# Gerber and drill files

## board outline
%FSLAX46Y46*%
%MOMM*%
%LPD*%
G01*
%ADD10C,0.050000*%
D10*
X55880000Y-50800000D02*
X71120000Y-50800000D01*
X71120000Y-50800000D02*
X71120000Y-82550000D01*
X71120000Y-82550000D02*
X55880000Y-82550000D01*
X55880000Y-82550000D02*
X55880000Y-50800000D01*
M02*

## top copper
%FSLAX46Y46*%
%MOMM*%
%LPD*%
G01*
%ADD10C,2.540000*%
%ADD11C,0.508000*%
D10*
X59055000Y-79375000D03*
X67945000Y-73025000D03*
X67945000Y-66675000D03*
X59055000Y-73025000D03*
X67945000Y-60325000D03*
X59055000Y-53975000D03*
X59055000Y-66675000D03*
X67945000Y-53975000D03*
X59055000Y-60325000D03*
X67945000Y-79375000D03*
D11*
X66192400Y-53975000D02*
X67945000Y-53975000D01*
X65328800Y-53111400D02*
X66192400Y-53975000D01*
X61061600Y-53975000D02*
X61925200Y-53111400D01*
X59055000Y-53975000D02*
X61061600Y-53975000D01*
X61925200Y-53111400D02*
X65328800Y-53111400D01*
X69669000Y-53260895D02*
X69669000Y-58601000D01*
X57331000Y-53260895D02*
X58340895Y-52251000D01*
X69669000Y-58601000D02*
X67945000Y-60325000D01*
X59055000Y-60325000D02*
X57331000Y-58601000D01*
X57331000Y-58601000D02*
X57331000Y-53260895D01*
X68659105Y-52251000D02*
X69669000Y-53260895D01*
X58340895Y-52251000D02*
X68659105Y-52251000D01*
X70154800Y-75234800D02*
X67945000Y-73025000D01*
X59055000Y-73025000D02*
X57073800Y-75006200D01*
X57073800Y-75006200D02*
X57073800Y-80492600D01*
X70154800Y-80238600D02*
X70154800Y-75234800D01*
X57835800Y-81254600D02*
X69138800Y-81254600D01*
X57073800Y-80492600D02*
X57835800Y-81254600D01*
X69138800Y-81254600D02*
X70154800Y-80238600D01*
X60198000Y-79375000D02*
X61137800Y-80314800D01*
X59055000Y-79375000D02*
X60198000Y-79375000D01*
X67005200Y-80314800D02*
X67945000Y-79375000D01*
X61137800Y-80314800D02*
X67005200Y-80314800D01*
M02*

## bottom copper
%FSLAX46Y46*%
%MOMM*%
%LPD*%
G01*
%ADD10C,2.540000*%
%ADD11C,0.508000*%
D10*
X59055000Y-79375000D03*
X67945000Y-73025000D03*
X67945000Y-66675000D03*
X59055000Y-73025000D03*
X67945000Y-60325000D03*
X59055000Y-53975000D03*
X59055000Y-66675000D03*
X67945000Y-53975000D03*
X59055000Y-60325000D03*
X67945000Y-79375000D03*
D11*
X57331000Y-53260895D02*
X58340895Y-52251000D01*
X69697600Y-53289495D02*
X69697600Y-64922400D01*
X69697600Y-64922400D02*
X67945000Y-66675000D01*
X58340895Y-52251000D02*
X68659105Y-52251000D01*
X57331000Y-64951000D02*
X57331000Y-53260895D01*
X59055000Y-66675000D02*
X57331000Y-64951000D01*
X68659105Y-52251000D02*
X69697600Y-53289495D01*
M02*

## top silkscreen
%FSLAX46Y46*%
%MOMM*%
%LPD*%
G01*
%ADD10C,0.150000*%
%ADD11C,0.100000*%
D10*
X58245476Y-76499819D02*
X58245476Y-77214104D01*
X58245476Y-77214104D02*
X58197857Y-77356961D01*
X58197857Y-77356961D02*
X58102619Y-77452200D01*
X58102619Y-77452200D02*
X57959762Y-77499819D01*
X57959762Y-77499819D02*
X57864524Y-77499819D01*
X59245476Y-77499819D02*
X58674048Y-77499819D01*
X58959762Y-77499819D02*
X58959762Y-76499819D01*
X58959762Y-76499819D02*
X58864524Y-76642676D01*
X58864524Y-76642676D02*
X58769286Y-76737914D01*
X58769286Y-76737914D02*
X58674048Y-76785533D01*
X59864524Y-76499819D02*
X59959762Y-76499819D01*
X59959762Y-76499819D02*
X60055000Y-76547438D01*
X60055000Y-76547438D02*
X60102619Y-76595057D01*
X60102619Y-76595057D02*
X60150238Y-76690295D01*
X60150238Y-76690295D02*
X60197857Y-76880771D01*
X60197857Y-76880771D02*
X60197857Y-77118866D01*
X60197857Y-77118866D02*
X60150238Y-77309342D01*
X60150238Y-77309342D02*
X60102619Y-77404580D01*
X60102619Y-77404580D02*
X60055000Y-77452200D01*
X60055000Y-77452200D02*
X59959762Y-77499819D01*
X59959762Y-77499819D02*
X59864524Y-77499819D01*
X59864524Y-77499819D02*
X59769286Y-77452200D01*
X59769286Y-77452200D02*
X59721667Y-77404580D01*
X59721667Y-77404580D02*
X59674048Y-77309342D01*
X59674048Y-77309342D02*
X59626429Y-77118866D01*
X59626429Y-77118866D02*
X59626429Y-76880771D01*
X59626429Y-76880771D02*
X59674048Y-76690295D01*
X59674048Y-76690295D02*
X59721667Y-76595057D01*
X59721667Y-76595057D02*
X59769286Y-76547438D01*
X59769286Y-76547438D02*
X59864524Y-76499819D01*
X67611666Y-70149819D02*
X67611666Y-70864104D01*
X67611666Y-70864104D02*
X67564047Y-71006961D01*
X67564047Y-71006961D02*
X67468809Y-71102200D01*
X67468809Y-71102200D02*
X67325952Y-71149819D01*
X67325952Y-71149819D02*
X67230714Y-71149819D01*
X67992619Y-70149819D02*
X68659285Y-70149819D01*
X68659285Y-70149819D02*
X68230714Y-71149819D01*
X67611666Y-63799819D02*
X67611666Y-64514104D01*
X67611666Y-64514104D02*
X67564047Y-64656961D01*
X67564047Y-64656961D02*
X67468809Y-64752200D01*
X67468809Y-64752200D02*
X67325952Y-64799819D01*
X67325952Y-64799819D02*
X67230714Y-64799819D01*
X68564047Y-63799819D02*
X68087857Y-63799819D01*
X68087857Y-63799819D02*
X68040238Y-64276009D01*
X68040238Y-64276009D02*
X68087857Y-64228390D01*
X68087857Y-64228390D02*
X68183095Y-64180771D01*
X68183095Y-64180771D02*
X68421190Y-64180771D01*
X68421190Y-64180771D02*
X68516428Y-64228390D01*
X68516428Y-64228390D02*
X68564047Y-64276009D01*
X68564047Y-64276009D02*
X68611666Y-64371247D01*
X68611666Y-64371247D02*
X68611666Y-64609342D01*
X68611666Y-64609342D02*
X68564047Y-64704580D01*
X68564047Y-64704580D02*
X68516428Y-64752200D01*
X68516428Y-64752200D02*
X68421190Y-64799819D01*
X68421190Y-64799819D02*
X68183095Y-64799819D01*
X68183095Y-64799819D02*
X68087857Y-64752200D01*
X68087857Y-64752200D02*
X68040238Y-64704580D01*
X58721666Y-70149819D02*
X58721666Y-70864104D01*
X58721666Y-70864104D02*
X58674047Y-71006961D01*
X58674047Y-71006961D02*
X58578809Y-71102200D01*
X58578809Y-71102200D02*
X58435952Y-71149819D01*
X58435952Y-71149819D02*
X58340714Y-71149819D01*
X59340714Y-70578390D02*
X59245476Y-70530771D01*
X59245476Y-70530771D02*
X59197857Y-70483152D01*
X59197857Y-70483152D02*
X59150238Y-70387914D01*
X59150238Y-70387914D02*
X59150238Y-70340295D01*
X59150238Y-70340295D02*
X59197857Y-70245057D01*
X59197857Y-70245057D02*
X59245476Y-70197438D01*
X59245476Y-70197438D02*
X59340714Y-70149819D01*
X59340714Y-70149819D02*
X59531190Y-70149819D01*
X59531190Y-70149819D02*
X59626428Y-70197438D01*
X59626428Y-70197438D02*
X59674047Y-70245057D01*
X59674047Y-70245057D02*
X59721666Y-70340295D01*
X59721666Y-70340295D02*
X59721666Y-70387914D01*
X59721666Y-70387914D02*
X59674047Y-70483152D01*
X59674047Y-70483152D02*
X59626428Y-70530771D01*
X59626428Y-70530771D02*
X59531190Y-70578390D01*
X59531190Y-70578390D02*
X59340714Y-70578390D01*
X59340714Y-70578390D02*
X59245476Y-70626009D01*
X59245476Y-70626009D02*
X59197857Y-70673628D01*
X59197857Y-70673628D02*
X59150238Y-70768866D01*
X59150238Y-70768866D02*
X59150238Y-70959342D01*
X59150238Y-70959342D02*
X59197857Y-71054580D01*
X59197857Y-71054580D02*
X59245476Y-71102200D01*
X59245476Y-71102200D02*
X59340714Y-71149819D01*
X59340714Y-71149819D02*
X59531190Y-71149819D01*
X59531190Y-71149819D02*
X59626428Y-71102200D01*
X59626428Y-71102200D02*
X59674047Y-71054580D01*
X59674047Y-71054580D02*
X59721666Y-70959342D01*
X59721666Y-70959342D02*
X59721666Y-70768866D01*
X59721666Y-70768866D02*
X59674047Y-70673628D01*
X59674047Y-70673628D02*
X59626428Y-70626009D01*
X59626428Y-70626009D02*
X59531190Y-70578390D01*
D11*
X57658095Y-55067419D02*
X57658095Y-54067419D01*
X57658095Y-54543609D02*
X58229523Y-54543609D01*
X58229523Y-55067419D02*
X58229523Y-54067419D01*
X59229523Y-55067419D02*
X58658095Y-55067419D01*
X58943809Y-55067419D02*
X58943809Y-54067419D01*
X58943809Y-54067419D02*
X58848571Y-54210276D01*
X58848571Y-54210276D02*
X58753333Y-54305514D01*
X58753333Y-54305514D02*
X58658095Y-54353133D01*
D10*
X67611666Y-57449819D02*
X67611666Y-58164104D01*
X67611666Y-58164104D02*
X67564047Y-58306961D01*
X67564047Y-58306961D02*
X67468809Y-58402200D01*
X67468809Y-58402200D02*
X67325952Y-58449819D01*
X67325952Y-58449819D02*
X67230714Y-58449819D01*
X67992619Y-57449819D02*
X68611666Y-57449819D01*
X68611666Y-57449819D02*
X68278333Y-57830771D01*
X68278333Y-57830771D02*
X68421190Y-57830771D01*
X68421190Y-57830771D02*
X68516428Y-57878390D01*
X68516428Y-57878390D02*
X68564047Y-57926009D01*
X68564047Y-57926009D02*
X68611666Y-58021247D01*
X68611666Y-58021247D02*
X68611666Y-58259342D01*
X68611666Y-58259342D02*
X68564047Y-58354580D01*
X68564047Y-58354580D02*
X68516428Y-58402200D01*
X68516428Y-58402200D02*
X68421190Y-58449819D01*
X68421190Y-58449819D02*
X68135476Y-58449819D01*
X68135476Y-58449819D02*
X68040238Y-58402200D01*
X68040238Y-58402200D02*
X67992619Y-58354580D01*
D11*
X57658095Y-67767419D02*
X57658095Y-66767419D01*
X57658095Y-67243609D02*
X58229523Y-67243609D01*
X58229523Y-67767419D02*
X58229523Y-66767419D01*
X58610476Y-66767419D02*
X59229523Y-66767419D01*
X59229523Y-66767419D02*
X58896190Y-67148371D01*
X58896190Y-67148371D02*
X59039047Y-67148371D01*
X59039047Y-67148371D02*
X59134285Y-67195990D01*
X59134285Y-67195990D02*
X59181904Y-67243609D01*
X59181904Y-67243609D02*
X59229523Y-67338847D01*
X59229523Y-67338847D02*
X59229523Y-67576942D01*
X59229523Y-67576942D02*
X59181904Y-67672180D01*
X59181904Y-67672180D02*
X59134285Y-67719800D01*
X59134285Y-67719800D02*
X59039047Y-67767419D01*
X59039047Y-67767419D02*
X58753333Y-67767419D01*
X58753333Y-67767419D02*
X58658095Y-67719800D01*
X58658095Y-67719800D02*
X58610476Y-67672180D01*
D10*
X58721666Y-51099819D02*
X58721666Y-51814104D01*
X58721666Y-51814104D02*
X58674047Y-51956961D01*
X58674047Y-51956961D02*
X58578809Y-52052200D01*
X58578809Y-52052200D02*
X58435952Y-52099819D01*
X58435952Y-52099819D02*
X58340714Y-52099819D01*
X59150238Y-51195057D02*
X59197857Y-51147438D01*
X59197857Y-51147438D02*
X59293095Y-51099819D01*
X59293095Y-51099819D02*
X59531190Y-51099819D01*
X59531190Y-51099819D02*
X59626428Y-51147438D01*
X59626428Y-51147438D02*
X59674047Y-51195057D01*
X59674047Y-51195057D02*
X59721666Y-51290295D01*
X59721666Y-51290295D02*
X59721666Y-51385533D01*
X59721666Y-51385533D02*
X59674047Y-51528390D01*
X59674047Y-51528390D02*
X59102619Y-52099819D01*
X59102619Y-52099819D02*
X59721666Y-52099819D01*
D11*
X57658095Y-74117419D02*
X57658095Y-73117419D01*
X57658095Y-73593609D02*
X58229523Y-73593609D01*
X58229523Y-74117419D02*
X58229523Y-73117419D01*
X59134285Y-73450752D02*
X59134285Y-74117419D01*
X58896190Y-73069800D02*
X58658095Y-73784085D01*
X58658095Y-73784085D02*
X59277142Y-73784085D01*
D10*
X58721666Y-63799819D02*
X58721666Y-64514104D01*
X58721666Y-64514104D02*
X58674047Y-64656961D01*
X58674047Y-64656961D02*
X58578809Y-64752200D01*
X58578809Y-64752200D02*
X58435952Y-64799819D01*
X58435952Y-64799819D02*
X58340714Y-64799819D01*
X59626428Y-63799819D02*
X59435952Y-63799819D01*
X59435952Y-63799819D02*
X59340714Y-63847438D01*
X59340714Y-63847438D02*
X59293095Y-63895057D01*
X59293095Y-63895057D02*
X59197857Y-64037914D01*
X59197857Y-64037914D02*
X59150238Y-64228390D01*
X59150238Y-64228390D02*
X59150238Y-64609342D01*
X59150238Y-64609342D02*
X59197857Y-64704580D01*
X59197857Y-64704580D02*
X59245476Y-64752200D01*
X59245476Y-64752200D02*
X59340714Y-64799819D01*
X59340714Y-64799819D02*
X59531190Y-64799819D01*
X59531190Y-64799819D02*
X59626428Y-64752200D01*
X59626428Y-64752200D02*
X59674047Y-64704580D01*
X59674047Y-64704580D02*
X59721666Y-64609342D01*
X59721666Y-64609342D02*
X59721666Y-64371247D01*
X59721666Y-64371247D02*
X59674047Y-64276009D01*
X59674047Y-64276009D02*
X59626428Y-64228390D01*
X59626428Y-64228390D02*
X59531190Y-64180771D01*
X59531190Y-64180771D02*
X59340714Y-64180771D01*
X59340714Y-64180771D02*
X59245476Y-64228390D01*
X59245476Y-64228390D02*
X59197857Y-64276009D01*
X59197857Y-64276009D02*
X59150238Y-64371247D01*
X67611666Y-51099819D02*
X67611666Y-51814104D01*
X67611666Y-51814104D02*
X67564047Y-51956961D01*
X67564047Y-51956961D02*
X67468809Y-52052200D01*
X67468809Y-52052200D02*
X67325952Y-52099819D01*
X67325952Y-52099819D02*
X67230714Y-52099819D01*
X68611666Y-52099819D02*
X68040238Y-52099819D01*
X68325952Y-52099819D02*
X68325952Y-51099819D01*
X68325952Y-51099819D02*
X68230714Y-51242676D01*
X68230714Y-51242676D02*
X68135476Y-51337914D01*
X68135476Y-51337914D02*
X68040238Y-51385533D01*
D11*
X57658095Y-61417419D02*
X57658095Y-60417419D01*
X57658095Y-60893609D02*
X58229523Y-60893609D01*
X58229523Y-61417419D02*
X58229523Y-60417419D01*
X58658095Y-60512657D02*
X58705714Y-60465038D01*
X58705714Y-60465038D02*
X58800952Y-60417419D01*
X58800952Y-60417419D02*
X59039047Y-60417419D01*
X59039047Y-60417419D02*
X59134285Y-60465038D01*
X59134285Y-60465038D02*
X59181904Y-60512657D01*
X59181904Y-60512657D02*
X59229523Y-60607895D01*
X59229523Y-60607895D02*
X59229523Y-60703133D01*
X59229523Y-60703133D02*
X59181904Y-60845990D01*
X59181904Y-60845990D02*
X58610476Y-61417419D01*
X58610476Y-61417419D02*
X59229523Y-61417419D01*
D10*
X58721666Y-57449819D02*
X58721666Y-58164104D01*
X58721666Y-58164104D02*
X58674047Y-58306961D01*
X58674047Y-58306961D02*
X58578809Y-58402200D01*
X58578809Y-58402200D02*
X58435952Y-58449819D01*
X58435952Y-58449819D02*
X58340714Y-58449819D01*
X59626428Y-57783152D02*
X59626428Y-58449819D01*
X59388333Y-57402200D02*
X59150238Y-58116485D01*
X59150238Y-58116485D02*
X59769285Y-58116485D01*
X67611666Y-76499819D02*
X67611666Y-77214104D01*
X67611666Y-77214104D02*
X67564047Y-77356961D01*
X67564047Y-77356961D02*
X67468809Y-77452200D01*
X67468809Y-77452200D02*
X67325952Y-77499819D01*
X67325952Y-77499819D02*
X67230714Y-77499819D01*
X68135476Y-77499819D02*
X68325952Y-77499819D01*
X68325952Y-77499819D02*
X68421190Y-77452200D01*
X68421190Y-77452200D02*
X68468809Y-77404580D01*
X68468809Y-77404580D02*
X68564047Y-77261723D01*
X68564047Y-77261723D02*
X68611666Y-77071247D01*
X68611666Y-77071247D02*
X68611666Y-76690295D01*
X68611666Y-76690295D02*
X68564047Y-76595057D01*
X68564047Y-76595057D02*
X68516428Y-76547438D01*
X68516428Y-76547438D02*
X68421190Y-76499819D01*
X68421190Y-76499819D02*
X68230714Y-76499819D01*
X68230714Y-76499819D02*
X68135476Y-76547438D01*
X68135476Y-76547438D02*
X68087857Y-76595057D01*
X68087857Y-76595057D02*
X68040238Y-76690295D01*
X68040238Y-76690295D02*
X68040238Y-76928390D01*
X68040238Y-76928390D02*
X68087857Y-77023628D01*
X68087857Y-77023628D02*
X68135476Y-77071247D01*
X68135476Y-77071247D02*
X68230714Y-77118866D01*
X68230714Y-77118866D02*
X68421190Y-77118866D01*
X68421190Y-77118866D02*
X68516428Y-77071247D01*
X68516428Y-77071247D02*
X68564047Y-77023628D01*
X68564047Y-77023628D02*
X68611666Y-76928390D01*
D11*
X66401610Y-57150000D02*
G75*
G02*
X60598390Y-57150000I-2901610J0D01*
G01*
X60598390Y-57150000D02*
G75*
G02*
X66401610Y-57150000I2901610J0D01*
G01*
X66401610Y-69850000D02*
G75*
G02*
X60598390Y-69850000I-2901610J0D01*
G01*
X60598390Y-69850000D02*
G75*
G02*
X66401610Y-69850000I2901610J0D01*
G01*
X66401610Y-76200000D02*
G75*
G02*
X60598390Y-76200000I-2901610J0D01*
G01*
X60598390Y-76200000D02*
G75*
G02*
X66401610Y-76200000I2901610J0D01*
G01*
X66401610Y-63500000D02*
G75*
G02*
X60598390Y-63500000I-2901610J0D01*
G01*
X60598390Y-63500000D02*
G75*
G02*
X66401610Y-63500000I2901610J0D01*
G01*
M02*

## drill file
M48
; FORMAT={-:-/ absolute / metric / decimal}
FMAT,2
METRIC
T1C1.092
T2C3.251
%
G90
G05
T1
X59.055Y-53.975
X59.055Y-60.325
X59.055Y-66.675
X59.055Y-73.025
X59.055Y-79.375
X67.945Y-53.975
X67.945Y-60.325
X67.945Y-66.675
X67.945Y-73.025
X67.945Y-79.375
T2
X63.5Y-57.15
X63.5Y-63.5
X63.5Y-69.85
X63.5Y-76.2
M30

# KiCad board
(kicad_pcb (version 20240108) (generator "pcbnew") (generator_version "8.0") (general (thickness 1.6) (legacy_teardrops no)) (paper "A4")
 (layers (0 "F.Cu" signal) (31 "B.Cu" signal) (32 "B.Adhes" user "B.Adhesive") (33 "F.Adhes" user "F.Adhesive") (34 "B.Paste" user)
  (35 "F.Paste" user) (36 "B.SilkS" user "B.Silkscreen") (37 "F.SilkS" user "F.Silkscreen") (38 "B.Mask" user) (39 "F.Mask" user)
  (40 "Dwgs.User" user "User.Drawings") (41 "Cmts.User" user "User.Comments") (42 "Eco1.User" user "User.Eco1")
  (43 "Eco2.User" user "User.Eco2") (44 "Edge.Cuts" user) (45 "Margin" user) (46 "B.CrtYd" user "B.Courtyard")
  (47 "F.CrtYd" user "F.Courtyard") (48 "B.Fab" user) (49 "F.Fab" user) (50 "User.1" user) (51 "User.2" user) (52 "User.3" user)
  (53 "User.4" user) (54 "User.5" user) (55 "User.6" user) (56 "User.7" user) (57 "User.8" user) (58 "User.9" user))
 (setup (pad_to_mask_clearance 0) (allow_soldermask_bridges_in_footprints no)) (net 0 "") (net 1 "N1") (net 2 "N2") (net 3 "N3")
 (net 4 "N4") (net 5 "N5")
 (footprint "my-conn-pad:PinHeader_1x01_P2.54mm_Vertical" (layer "F.Cu") (at 59.055 79.375)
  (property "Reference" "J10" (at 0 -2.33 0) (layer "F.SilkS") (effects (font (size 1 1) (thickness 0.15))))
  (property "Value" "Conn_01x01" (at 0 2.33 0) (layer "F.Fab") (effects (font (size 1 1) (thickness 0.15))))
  (pad "1" thru_hole circle (at 0 0) (size 2.54 2.54) (drill 1.0922) (layers "*.Cu" "*.Mask") (remove_unused_layers no) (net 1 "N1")))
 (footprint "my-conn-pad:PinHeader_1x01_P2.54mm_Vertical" (layer "F.Cu") (at 67.945 73.025)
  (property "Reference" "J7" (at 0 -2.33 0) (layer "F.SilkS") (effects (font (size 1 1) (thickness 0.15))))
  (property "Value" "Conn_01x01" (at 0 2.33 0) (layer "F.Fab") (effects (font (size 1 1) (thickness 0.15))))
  (pad "1" thru_hole circle (at 0 0) (size 2.54 2.54) (drill 1.0922) (layers "*.Cu" "*.Mask") (remove_unused_layers no) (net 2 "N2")))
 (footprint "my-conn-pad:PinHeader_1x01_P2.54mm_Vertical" (layer "F.Cu") (at 67.945 66.675)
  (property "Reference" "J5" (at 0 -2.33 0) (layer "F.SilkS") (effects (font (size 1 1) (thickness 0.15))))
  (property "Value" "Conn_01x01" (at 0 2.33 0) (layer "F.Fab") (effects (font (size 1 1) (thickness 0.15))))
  (pad "1" thru_hole circle (at 0 0) (size 2.54 2.54) (drill 1.0922) (layers "*.Cu" "*.Mask") (remove_unused_layers no) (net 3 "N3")))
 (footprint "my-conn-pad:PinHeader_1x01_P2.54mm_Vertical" (layer "F.Cu") (at 59.055 73.025)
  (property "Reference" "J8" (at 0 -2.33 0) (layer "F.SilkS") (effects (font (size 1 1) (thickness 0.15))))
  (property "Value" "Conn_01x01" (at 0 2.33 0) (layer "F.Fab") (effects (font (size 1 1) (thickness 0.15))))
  (pad "1" thru_hole circle (at 0 0) (size 2.54 2.54) (drill 1.0922) (layers "*.Cu" "*.Mask") (remove_unused_layers no) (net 2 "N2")))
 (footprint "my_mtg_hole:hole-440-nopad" (layer "F.Cu") (at 63.5 57.15)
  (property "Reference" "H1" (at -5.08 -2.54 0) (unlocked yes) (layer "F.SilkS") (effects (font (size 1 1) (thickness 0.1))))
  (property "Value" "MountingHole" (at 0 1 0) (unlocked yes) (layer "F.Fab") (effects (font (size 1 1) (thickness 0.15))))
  (fp_circle (center 0 0) (end 1.143 2.667) (stroke (width 0.1) (type default)) (fill none) (layer "F.SilkS"))
  (pad "" np_thru_hole circle (at 0 0) (size 1.524 1.524) (drill 3.2512) (layers "F&B.Cu" "*.Mask")))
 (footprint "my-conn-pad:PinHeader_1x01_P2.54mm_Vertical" (layer "F.Cu") (at 67.945 60.325)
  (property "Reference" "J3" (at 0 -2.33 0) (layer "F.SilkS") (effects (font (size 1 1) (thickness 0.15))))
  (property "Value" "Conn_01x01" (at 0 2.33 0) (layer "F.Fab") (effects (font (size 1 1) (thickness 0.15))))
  (pad "1" thru_hole circle (at 0 0) (size 2.54 2.54) (drill 1.0922) (layers "*.Cu" "*.Mask") (remove_unused_layers no) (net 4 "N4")))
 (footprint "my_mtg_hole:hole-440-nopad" (layer "F.Cu") (at 63.5 69.85)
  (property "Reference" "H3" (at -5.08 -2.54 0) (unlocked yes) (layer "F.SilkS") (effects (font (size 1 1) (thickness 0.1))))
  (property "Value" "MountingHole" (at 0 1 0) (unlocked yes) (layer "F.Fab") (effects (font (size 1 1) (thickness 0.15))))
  (fp_circle (center 0 0) (end 1.143 2.667) (stroke (width 0.1) (type default)) (fill none) (layer "F.SilkS"))
  (pad "" np_thru_hole circle (at 0 0) (size 1.524 1.524) (drill 3.2512) (layers "F&B.Cu" "*.Mask")))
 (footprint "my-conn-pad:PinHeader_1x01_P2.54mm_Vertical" (layer "F.Cu") (at 59.055 53.975)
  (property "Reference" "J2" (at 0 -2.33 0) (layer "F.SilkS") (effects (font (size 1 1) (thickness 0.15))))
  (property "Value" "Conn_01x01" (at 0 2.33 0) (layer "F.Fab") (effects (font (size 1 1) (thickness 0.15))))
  (pad "1" thru_hole circle (at 0 0) (size 2.54 2.54) (drill 1.0922) (layers "*.Cu" "*.Mask") (remove_unused_layers no) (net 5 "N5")))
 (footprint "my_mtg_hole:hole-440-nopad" (layer "F.Cu") (at 63.5 76.2)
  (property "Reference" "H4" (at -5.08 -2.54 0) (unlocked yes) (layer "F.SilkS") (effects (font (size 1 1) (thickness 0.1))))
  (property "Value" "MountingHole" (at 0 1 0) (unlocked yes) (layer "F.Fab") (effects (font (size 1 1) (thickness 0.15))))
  (fp_circle (center 0 0) (end 1.143 2.667) (stroke (width 0.1) (type default)) (fill none) (layer "F.SilkS"))
  (pad "" np_thru_hole circle (at 0 0) (size 1.524 1.524) (drill 3.2512) (layers "F&B.Cu" "*.Mask")))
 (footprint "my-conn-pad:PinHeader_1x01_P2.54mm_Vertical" (layer "F.Cu") (at 59.055 66.675)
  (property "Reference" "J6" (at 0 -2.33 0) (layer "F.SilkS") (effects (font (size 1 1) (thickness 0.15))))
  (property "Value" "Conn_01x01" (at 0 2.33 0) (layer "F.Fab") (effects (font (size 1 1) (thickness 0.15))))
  (pad "1" thru_hole circle (at 0 0) (size 2.54 2.54) (drill 1.0922) (layers "*.Cu" "*.Mask") (remove_unused_layers no) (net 3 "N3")))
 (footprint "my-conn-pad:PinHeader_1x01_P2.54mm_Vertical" (layer "F.Cu") (at 67.945 53.975)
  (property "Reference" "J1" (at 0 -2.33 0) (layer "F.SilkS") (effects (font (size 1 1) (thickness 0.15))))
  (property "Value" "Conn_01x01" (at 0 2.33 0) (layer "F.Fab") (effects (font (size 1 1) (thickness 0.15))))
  (pad "1" thru_hole circle (at 0 0) (size 2.54 2.54) (drill 1.0922) (layers "*.Cu" "*.Mask") (remove_unused_layers no) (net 5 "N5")))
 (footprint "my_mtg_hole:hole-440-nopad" (layer "F.Cu") (at 63.5 63.5)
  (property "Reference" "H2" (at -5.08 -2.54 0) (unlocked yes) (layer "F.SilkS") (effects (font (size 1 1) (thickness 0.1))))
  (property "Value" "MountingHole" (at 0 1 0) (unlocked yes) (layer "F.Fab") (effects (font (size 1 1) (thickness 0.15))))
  (fp_circle (center 0 0) (end 1.143 2.667) (stroke (width 0.1) (type default)) (fill none) (layer "F.SilkS"))
  (pad "" np_thru_hole circle (at 0 0) (size 1.524 1.524) (drill 3.2512) (layers "F&B.Cu" "*.Mask")))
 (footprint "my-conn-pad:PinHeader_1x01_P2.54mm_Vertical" (layer "F.Cu") (at 59.055 60.325)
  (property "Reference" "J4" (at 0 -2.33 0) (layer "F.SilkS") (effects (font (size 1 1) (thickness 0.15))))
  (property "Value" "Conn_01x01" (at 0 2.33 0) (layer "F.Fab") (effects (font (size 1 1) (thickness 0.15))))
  (pad "1" thru_hole circle (at 0 0) (size 2.54 2.54) (drill 1.0922) (layers "*.Cu" "*.Mask") (remove_unused_layers no) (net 4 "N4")))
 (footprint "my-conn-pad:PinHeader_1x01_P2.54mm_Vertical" (layer "F.Cu") (at 67.945 79.375)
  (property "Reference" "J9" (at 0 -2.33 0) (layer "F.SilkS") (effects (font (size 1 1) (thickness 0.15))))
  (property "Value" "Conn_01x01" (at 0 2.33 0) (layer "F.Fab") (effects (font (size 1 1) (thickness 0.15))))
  (pad "1" thru_hole circle (at 0 0) (size 2.54 2.54) (drill 1.0922) (layers "*.Cu" "*.Mask") (remove_unused_layers no) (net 1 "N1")))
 (gr_line (start 55.88 50.8) (end 71.12 50.8) (stroke (width 0.05) (type default)) (layer "Edge.Cuts"))
 (gr_line (start 71.12 50.8) (end 71.12 82.55) (stroke (width 0.05) (type default)) (layer "Edge.Cuts"))
 (gr_line (start 71.12 82.55) (end 55.88 82.55) (stroke (width 0.05) (type default)) (layer "Edge.Cuts"))
 (gr_line (start 55.88 82.55) (end 55.88 50.8) (stroke (width 0.05) (type default)) (layer "Edge.Cuts"))
 (segment (start 66.1924 53.975) (end 67.945 53.975) (width 0.508) (layer "F.Cu") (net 5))
 (segment (start 65.3288 53.1114) (end 66.1924 53.975) (width 0.508) (layer "F.Cu") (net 5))
 (segment (start 61.0616 53.975) (end 61.9252 53.1114) (width 0.508) (layer "F.Cu") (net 5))
 (segment (start 59.055 53.975) (end 61.0616 53.975) (width 0.508) (layer "F.Cu") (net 5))
 (segment (start 61.9252 53.1114) (end 65.3288 53.1114) (width 0.508) (layer "F.Cu") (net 5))
 (segment (start 69.669 53.260895) (end 69.669 58.601) (width 0.508) (layer "F.Cu") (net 4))
 (segment (start 57.331 53.260895) (end 58.340895 52.251) (width 0.508) (layer "F.Cu") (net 4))
 (segment (start 69.669 58.601) (end 67.945 60.325) (width 0.508) (layer "F.Cu") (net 4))
 (segment (start 59.055 60.325) (end 57.331 58.601) (width 0.508) (layer "F.Cu") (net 4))
 (segment (start 57.331 58.601) (end 57.331 53.260895) (width 0.508) (layer "F.Cu") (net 4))
 (segment (start 68.659105 52.251) (end 69.669 53.260895) (width 0.508) (layer "F.Cu") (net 4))
 (segment (start 58.340895 52.251) (end 68.659105 52.251) (width 0.508) (layer "F.Cu") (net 4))
 (segment (start 57.331 53.260895) (end 58.340895 52.251) (width 0.508) (layer "B.Cu") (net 3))
 (segment (start 69.6976 53.289495) (end 69.6976 64.9224) (width 0.508) (layer "B.Cu") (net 3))
 (segment (start 69.6976 64.9224) (end 67.945 66.675) (width 0.508) (layer "B.Cu") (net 3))
 (segment (start 58.340895 52.251) (end 68.659105 52.251) (width 0.508) (layer "B.Cu") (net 3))
 (segment (start 57.331 64.951) (end 57.331 53.260895) (width 0.508) (layer "B.Cu") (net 3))
 (segment (start 59.055 66.675) (end 57.331 64.951) (width 0.508) (layer "B.Cu") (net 3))
 (segment (start 68.659105 52.251) (end 69.6976 53.289495) (width 0.508) (layer "B.Cu") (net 3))
 (segment (start 70.1548 75.2348) (end 67.945 73.025) (width 0.508) (layer "F.Cu") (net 2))
 (segment (start 59.055 73.025) (end 57.0738 75.0062) (width 0.508) (layer "F.Cu") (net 2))
 (segment (start 57.0738 75.0062) (end 57.0738 80.4926) (width 0.508) (layer "F.Cu") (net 2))
 (segment (start 70.1548 80.2386) (end 70.1548 75.2348) (width 0.508) (layer "F.Cu") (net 2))
 (segment (start 57.8358 81.2546) (end 69.1388 81.2546) (width 0.508) (layer "F.Cu") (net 2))
 (segment (start 57.0738 80.4926) (end 57.8358 81.2546) (width 0.508) (layer "F.Cu") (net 2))
 (segment (start 69.1388 81.2546) (end 70.1548 80.2386) (width 0.508) (layer "F.Cu") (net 2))
 (segment (start 60.198 79.375) (end 61.1378 80.3148) (width 0.508) (layer "F.Cu") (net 1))
 (segment (start 59.055 79.375) (end 60.198 79.375) (width 0.508) (layer "F.Cu") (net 1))
 (segment (start 67.0052 80.3148) (end 67.945 79.375) (width 0.508) (layer "F.Cu") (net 1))
 (segment (start 61.1378 80.3148) (end 67.0052 80.3148) (width 0.508) (layer "F.Cu") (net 1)))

